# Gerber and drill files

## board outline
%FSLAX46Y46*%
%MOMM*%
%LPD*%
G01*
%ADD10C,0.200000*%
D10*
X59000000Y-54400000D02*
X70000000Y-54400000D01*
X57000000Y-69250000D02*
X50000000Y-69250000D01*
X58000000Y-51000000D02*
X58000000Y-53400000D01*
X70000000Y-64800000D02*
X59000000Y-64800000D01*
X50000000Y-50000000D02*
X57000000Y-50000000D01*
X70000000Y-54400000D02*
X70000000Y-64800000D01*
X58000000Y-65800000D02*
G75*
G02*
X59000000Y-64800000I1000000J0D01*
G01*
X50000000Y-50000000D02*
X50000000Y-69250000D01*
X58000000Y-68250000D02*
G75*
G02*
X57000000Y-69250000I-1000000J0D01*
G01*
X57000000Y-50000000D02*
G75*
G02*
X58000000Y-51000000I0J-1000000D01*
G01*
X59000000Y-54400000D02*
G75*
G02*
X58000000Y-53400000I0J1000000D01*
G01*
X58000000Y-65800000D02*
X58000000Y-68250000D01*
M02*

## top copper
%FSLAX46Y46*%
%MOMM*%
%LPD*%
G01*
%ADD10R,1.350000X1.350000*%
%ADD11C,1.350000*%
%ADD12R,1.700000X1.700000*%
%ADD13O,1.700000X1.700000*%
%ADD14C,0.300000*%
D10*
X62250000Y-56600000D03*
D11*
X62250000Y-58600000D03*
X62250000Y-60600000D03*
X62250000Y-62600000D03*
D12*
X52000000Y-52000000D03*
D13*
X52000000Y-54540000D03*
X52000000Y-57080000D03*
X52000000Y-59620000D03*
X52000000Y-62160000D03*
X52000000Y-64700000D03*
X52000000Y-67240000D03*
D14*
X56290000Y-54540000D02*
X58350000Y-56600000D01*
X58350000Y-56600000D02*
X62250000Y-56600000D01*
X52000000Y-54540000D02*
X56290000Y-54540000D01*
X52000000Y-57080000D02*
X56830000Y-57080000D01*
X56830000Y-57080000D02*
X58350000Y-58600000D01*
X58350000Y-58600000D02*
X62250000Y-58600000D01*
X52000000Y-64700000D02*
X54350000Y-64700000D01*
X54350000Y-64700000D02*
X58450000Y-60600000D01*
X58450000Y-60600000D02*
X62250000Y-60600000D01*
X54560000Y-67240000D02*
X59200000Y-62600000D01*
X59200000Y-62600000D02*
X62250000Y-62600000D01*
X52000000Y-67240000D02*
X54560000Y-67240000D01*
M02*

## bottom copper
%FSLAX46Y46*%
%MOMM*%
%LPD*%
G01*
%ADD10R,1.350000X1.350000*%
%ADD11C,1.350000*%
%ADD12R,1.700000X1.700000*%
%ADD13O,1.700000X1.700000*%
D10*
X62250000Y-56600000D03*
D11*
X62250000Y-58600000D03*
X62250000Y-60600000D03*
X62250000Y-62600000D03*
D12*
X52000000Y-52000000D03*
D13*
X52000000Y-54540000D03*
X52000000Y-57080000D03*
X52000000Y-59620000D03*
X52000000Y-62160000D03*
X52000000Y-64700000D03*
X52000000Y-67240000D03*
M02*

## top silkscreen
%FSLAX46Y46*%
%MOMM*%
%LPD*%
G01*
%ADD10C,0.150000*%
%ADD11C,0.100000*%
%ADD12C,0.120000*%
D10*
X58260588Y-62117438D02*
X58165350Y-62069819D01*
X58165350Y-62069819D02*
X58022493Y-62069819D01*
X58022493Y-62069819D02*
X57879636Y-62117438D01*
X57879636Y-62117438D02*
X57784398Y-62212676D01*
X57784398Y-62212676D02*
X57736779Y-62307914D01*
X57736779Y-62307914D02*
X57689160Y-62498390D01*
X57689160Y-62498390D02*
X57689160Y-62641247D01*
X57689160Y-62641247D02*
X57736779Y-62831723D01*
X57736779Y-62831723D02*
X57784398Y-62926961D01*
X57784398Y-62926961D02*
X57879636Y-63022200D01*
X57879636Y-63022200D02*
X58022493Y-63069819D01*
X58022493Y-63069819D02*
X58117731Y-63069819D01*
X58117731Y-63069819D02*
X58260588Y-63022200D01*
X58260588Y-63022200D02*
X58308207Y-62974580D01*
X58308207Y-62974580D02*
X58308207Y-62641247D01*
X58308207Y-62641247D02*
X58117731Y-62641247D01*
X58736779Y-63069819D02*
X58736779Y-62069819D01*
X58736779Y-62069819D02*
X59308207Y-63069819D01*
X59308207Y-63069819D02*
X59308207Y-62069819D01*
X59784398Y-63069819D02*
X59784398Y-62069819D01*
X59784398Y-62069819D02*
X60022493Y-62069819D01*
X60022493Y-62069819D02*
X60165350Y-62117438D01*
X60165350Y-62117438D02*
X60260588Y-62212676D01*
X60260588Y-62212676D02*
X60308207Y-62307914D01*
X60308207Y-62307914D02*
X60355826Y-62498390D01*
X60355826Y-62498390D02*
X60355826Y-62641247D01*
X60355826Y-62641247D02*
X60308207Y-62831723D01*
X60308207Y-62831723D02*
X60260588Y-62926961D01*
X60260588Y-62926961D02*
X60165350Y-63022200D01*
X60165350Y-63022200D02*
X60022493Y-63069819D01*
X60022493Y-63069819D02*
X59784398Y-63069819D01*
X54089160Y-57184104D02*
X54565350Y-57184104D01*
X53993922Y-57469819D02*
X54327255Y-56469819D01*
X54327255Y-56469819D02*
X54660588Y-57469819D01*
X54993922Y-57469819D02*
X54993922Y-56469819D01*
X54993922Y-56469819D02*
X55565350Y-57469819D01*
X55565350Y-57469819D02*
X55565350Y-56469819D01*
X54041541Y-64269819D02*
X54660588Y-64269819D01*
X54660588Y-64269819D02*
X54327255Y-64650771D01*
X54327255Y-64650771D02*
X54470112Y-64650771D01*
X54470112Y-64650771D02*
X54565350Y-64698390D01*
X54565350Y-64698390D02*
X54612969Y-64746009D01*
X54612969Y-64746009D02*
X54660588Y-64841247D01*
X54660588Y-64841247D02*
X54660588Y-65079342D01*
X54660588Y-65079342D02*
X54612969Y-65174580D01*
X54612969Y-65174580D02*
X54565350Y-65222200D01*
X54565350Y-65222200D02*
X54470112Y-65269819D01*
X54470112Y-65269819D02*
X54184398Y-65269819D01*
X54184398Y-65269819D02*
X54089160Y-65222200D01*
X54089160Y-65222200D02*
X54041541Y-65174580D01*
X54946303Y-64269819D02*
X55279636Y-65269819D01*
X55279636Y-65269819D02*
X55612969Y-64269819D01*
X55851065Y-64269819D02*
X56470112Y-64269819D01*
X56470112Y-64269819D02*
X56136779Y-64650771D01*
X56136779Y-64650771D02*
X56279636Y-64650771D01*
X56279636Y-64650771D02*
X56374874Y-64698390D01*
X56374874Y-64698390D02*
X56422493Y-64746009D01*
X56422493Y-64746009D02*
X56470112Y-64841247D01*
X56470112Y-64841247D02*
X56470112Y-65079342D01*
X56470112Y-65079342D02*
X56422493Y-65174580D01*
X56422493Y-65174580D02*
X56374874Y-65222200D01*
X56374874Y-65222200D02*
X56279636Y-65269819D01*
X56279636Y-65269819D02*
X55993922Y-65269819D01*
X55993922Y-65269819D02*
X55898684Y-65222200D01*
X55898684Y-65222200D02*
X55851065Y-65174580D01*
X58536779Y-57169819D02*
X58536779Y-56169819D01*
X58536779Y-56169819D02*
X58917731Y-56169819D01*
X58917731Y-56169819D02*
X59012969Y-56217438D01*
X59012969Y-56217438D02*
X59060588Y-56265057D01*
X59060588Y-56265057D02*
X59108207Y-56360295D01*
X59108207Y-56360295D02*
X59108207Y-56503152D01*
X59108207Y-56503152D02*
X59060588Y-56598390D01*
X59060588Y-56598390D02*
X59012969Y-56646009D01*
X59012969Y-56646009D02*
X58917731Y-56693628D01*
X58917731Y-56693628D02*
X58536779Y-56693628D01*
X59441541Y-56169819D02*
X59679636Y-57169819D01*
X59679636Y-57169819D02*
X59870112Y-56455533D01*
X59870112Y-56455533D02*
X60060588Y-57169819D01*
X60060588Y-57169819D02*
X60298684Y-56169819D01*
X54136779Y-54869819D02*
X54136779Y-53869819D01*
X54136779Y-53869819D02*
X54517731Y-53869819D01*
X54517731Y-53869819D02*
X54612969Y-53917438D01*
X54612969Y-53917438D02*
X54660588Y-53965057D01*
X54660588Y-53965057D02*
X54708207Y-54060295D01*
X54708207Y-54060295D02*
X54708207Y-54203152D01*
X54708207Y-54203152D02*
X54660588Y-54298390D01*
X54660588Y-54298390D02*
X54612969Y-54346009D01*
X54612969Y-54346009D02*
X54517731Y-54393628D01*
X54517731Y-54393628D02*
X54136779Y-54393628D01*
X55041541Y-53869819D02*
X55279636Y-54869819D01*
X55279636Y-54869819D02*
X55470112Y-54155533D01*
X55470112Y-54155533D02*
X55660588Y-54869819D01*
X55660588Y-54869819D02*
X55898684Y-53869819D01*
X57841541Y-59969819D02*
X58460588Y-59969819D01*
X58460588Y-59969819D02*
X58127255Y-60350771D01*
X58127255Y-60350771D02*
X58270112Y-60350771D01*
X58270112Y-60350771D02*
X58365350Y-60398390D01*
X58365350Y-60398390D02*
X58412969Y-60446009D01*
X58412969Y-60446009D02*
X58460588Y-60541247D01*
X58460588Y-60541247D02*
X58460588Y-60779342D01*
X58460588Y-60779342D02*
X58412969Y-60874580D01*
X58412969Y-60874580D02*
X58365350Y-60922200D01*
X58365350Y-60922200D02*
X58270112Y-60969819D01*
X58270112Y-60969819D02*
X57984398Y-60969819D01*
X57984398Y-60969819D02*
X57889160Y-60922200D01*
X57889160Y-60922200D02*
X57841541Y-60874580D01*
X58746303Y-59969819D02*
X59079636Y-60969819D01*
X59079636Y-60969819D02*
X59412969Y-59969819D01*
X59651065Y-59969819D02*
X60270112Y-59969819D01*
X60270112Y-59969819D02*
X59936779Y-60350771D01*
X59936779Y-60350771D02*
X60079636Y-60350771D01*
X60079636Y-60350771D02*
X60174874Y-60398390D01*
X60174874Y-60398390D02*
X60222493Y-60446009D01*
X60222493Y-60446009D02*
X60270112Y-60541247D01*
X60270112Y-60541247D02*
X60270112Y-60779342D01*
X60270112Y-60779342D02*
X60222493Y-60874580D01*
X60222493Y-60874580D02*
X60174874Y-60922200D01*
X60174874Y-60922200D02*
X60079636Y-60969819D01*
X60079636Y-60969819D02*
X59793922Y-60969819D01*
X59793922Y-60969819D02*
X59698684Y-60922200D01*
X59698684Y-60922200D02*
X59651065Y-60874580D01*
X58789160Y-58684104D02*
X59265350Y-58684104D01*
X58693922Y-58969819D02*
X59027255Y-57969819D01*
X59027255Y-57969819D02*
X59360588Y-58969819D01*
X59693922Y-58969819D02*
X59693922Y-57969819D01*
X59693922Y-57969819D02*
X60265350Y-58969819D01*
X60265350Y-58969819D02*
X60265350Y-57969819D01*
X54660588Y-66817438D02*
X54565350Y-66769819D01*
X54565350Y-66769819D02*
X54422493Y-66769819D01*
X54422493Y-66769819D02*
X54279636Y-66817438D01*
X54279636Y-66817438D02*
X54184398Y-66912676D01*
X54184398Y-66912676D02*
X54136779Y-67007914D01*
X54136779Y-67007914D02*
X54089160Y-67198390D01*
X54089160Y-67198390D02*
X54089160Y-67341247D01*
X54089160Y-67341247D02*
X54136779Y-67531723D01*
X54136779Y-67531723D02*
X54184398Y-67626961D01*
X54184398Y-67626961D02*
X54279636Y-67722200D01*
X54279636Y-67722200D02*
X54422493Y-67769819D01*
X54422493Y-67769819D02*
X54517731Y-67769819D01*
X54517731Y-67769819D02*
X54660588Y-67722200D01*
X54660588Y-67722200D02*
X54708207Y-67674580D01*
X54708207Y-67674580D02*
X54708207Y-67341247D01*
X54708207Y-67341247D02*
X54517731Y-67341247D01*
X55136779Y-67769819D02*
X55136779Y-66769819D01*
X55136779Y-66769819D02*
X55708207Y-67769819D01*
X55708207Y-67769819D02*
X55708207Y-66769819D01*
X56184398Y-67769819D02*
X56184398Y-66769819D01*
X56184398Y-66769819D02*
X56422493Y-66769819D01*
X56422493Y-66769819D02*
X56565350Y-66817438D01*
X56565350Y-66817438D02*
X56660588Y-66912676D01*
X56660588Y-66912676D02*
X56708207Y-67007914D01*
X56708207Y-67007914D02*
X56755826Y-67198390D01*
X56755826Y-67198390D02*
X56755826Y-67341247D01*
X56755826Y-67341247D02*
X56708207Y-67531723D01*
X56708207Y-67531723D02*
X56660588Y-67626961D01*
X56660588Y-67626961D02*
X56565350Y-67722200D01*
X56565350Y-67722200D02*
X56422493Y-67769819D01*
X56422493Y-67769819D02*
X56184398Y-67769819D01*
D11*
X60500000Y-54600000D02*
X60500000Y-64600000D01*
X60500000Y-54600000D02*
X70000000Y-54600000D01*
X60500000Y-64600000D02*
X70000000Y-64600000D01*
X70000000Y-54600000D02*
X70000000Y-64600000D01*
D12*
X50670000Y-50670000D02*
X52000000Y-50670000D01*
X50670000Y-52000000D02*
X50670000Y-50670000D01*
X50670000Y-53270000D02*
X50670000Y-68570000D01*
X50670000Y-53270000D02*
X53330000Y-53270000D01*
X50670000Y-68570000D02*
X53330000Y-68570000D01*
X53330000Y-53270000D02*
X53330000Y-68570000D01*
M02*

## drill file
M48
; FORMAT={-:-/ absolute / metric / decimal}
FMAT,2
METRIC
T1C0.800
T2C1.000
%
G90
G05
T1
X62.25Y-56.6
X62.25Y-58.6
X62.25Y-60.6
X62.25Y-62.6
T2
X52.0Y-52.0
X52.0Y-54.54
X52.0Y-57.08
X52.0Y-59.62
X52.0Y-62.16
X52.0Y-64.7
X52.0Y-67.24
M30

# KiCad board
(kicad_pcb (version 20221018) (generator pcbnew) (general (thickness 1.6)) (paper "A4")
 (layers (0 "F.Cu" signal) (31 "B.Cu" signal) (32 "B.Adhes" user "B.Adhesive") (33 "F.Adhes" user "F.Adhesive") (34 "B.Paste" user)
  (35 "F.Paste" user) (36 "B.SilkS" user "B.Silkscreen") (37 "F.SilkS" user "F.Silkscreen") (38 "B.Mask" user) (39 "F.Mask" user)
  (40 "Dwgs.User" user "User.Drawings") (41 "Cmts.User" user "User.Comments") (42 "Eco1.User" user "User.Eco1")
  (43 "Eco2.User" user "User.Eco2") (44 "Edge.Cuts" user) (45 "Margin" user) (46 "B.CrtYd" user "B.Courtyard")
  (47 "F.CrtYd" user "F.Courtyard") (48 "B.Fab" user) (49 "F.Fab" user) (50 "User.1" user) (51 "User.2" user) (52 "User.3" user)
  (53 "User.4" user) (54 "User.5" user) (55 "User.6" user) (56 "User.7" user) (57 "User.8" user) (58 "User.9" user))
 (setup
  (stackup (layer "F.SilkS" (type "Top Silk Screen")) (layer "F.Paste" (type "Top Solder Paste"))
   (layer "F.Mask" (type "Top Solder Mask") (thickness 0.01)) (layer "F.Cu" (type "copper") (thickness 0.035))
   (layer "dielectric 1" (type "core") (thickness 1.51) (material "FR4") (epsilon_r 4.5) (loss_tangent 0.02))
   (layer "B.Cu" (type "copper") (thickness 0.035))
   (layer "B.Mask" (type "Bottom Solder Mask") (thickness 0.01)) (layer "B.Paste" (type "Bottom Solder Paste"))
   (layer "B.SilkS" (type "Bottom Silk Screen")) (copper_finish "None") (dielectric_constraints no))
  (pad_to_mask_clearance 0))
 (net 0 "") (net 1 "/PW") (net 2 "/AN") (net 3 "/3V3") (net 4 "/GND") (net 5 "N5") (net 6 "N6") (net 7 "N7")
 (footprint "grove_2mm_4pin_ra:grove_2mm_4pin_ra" (layer "F.Cu") (at 62.25 56.6)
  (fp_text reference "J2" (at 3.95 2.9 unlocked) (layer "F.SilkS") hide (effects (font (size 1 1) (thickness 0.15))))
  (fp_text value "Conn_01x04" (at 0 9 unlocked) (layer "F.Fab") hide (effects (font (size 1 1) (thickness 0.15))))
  (fp_line (start -1.75 -2) (end -1.75 8) (stroke (width 0.1) (type default)) (layer "F.SilkS"))
  (fp_line (start -1.75 -2) (end 7.75 -2) (stroke (width 0.1) (type default)) (layer "F.SilkS"))
  (fp_line (start -1.75 8) (end 7.75 8) (stroke (width 0.1) (type default)) (layer "F.SilkS"))
  (fp_line (start 7.75 -2) (end 7.75 8) (stroke (width 0.1) (type default)) (layer "F.SilkS"))
  (pad "1" thru_hole rect (at 0 0) (size 1.35 1.35) (drill 0.8) (layers "*.Cu" "*.Mask") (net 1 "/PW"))
  (pad "2" thru_hole circle (at 0 2) (size 1.35 1.35) (drill 0.8) (layers "*.Cu" "*.Mask") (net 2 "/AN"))
  (pad "3" thru_hole circle (at 0 4) (size 1.35 1.35) (drill 0.8) (layers "*.Cu" "*.Mask") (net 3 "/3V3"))
  (pad "4" thru_hole circle (at 0 6) (size 1.35 1.35) (drill 0.8) (layers "*.Cu" "*.Mask") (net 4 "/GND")))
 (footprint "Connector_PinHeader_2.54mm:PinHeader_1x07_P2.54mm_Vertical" (layer "F.Cu") (at 52 52)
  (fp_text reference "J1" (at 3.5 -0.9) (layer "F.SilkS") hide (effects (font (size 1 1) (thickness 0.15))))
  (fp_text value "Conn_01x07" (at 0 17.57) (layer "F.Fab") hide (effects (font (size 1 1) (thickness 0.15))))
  (fp_line (start -1.33 -1.33) (end 0 -1.33) (stroke (width 0.12) (type solid)) (layer "F.SilkS"))
  (fp_line (start -1.33 0) (end -1.33 -1.33) (stroke (width 0.12) (type solid)) (layer "F.SilkS"))
  (fp_line (start -1.33 1.27) (end -1.33 16.57) (stroke (width 0.12) (type solid)) (layer "F.SilkS"))
  (fp_line (start -1.33 1.27) (end 1.33 1.27) (stroke (width 0.12) (type solid)) (layer "F.SilkS"))
  (fp_line (start -1.33 16.57) (end 1.33 16.57) (stroke (width 0.12) (type solid)) (layer "F.SilkS"))
  (fp_line (start 1.33 1.27) (end 1.33 16.57) (stroke (width 0.12) (type solid)) (layer "F.SilkS"))
  (pad "1" thru_hole rect (at 0 0) (size 1.7 1.7) (drill 1) (layers "*.Cu" "*.Mask") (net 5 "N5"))
  (pad "2" thru_hole oval (at 0 2.54) (size 1.7 1.7) (drill 1) (layers "*.Cu" "*.Mask") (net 1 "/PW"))
  (pad "3" thru_hole oval (at 0 5.08) (size 1.7 1.7) (drill 1) (layers "*.Cu" "*.Mask") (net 2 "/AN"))
  (pad "4" thru_hole oval (at 0 7.62) (size 1.7 1.7) (drill 1) (layers "*.Cu" "*.Mask") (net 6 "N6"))
  (pad "5" thru_hole oval (at 0 10.16) (size 1.7 1.7) (drill 1) (layers "*.Cu" "*.Mask") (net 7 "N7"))
  (pad "6" thru_hole oval (at 0 12.7) (size 1.7 1.7) (drill 1) (layers "*.Cu" "*.Mask") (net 3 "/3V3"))
  (pad "7" thru_hole oval (at 0 15.24) (size 1.7 1.7) (drill 1) (layers "*.Cu" "*.Mask") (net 4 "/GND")))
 (gr_line (start 59 54.4) (end 70 54.4) (stroke (width 0.2) (type default)) (layer "Edge.Cuts"))
 (gr_line (start 57 69.25) (end 50 69.25) (stroke (width 0.2) (type default)) (layer "Edge.Cuts"))
 (gr_line (start 58 51) (end 58 53.4) (stroke (width 0.2) (type default)) (layer "Edge.Cuts"))
 (gr_line (start 70 64.8) (end 59 64.8) (stroke (width 0.2) (type default)) (layer "Edge.Cuts"))
 (gr_line (start 50 50) (end 57 50) (stroke (width 0.2) (type default)) (layer "Edge.Cuts"))
 (gr_line (start 70 54.4) (end 70 64.8) (stroke (width 0.2) (type default)) (layer "Edge.Cuts"))
 (gr_arc (start 58 65.8) (mid 58.292893 65.092893) (end 59 64.8) (stroke (width 0.2) (type default)) (layer "Edge.Cuts"))
 (gr_line (start 50 50) (end 50 69.25) (stroke (width 0.2) (type default)) (layer "Edge.Cuts"))
 (gr_arc (start 58 68.25) (mid 57.707107 68.957107) (end 57 69.25) (stroke (width 0.2) (type default)) (layer "Edge.Cuts"))
 (gr_arc (start 57 50) (mid 57.707107 50.292893) (end 58 51) (stroke (width 0.2) (type default)) (layer "Edge.Cuts"))
 (gr_arc (start 59 54.4) (mid 58.292893 54.107107) (end 58 53.4) (stroke (width 0.2) (type default)) (layer "Edge.Cuts"))
 (gr_line (start 58 65.8) (end 58 68.25) (stroke (width 0.2) (type default)) (layer "Edge.Cuts"))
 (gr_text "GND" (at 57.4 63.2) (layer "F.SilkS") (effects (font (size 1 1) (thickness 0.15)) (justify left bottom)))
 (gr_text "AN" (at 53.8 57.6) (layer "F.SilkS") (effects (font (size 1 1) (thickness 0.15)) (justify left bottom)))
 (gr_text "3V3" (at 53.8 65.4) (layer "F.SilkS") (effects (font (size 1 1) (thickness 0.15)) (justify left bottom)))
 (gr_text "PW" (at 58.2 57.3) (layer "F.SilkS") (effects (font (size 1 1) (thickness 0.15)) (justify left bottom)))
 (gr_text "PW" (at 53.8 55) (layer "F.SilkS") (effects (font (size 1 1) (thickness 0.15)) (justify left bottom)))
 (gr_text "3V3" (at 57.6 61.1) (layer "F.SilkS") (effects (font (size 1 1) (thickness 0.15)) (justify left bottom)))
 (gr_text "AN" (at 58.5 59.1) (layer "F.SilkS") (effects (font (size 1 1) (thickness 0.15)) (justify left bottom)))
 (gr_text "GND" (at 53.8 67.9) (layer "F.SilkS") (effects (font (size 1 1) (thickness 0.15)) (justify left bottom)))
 (segment (start 56.29 54.54) (end 58.35 56.6) (width 0.3) (layer "F.Cu") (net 1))
 (segment (start 58.35 56.6) (end 62.25 56.6) (width 0.3) (layer "F.Cu") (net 1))
 (segment (start 52 54.54) (end 56.29 54.54) (width 0.3) (layer "F.Cu") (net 1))
 (segment (start 52 57.08) (end 56.83 57.08) (width 0.3) (layer "F.Cu") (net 2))
 (segment (start 56.83 57.08) (end 58.35 58.6) (width 0.3) (layer "F.Cu") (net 2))
 (segment (start 58.35 58.6) (end 62.25 58.6) (width 0.3) (layer "F.Cu") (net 2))
 (segment (start 52 64.7) (end 54.35 64.7) (width 0.3) (layer "F.Cu") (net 3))
 (segment (start 54.35 64.7) (end 58.45 60.6) (width 0.3) (layer "F.Cu") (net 3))
 (segment (start 58.45 60.6) (end 62.25 60.6) (width 0.3) (layer "F.Cu") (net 3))
 (segment (start 54.56 67.24) (end 59.2 62.6) (width 0.3) (layer "F.Cu") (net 4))
 (segment (start 59.2 62.6) (end 62.25 62.6) (width 0.3) (layer "F.Cu") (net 4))
 (segment (start 52 67.24) (end 54.56 67.24) (width 0.3) (layer "F.Cu") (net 4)))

